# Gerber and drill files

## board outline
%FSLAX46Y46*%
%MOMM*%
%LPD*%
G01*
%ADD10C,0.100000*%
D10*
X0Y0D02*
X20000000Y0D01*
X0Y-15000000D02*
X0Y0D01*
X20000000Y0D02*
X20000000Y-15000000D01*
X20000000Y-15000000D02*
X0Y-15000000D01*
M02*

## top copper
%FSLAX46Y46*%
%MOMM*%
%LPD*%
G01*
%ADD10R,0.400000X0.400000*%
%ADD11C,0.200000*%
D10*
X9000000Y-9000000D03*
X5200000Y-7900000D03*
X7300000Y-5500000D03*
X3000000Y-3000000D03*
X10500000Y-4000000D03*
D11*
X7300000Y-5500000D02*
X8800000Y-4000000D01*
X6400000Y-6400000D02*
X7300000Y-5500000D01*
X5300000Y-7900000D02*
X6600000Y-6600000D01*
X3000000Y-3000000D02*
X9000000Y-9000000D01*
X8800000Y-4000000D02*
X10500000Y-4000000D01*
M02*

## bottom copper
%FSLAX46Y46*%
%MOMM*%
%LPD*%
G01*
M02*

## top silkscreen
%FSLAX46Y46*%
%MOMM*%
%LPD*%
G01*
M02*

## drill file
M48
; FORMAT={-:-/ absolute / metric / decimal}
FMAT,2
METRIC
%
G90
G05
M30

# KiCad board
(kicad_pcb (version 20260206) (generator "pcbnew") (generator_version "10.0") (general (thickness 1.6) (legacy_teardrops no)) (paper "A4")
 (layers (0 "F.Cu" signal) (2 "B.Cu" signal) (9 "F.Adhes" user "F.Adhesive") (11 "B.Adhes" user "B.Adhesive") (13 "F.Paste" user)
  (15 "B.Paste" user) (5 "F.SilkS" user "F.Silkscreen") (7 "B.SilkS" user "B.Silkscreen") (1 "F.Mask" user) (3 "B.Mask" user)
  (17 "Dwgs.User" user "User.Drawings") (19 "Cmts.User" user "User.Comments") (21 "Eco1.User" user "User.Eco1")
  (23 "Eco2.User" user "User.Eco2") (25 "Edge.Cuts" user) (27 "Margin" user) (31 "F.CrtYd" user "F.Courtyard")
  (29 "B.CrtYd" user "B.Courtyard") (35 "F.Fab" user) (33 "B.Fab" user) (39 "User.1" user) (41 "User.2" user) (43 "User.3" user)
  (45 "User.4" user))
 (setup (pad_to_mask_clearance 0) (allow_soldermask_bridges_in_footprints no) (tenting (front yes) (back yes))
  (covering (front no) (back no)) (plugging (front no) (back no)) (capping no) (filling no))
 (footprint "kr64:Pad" (layer "F.Cu") (at 9 9)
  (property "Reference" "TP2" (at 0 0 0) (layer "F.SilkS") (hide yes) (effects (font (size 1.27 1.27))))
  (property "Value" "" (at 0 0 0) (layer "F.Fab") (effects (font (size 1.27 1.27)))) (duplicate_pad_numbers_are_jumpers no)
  (pad "1" smd rect (at 0 0) (size 0.4 0.4) (layers "F.Cu" "F.Mask" "F.Paste") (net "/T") (thermal_bridge_angle 45)))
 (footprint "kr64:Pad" (layer "F.Cu") (at 5.2 7.9)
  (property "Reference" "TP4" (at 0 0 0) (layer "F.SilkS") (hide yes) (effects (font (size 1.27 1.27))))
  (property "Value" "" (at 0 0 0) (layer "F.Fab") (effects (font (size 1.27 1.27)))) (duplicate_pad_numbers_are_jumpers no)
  (pad "1" smd rect (at 0 0) (size 0.4 0.4) (layers "F.Cu" "F.Mask" "F.Paste") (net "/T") (thermal_bridge_angle 45)))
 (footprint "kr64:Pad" (layer "F.Cu") (at 7.3 5.5)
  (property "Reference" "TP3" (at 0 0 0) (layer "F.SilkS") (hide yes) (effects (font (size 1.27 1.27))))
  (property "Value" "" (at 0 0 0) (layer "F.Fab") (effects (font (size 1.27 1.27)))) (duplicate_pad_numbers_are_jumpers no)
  (pad "1" smd rect (at 0 0) (size 0.4 0.4) (layers "F.Cu" "F.Mask" "F.Paste") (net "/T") (thermal_bridge_angle 45)))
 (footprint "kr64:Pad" (layer "F.Cu") (at 3 3)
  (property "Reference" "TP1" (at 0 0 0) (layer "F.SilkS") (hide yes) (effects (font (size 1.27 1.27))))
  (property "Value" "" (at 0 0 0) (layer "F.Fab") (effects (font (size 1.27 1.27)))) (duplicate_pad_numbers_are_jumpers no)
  (pad "1" smd rect (at 0 0) (size 0.4 0.4) (layers "F.Cu" "F.Mask" "F.Paste") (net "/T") (thermal_bridge_angle 45)))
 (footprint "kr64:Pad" (layer "F.Cu") (at 10.5 4)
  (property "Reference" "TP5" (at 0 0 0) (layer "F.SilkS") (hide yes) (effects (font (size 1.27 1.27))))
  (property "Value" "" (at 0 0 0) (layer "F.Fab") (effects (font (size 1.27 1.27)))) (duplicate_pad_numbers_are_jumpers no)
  (pad "1" smd rect (at 0 0) (size 0.4 0.4) (layers "F.Cu" "F.Mask" "F.Paste") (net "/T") (thermal_bridge_angle 45)))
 (gr_line (start 0 0) (end 20 0) (stroke (width 0.1) (type default)) (layer "Edge.Cuts"))
 (gr_line (start 0 15) (end 0 0) (stroke (width 0.1) (type default)) (layer "Edge.Cuts"))
 (gr_line (start 20 0) (end 20 15) (stroke (width 0.1) (type default)) (layer "Edge.Cuts"))
 (gr_line (start 20 15) (end 0 15) (stroke (width 0.1) (type default)) (layer "Edge.Cuts"))
 (segment (start 7.3 5.5) (end 8.8 4) (width 0.2) (layer "F.Cu") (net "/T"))
 (segment (start 6.4 6.4) (end 7.3 5.5) (width 0.2) (layer "F.Cu") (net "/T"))
 (segment (start 5.3 7.9) (end 6.6 6.6) (width 0.2) (layer "F.Cu") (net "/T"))
 (segment (start 3 3) (end 9 9) (width 0.2) (layer "F.Cu") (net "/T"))
 (segment (start 8.8 4) (end 10.5 4) (width 0.2) (layer "F.Cu") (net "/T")))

